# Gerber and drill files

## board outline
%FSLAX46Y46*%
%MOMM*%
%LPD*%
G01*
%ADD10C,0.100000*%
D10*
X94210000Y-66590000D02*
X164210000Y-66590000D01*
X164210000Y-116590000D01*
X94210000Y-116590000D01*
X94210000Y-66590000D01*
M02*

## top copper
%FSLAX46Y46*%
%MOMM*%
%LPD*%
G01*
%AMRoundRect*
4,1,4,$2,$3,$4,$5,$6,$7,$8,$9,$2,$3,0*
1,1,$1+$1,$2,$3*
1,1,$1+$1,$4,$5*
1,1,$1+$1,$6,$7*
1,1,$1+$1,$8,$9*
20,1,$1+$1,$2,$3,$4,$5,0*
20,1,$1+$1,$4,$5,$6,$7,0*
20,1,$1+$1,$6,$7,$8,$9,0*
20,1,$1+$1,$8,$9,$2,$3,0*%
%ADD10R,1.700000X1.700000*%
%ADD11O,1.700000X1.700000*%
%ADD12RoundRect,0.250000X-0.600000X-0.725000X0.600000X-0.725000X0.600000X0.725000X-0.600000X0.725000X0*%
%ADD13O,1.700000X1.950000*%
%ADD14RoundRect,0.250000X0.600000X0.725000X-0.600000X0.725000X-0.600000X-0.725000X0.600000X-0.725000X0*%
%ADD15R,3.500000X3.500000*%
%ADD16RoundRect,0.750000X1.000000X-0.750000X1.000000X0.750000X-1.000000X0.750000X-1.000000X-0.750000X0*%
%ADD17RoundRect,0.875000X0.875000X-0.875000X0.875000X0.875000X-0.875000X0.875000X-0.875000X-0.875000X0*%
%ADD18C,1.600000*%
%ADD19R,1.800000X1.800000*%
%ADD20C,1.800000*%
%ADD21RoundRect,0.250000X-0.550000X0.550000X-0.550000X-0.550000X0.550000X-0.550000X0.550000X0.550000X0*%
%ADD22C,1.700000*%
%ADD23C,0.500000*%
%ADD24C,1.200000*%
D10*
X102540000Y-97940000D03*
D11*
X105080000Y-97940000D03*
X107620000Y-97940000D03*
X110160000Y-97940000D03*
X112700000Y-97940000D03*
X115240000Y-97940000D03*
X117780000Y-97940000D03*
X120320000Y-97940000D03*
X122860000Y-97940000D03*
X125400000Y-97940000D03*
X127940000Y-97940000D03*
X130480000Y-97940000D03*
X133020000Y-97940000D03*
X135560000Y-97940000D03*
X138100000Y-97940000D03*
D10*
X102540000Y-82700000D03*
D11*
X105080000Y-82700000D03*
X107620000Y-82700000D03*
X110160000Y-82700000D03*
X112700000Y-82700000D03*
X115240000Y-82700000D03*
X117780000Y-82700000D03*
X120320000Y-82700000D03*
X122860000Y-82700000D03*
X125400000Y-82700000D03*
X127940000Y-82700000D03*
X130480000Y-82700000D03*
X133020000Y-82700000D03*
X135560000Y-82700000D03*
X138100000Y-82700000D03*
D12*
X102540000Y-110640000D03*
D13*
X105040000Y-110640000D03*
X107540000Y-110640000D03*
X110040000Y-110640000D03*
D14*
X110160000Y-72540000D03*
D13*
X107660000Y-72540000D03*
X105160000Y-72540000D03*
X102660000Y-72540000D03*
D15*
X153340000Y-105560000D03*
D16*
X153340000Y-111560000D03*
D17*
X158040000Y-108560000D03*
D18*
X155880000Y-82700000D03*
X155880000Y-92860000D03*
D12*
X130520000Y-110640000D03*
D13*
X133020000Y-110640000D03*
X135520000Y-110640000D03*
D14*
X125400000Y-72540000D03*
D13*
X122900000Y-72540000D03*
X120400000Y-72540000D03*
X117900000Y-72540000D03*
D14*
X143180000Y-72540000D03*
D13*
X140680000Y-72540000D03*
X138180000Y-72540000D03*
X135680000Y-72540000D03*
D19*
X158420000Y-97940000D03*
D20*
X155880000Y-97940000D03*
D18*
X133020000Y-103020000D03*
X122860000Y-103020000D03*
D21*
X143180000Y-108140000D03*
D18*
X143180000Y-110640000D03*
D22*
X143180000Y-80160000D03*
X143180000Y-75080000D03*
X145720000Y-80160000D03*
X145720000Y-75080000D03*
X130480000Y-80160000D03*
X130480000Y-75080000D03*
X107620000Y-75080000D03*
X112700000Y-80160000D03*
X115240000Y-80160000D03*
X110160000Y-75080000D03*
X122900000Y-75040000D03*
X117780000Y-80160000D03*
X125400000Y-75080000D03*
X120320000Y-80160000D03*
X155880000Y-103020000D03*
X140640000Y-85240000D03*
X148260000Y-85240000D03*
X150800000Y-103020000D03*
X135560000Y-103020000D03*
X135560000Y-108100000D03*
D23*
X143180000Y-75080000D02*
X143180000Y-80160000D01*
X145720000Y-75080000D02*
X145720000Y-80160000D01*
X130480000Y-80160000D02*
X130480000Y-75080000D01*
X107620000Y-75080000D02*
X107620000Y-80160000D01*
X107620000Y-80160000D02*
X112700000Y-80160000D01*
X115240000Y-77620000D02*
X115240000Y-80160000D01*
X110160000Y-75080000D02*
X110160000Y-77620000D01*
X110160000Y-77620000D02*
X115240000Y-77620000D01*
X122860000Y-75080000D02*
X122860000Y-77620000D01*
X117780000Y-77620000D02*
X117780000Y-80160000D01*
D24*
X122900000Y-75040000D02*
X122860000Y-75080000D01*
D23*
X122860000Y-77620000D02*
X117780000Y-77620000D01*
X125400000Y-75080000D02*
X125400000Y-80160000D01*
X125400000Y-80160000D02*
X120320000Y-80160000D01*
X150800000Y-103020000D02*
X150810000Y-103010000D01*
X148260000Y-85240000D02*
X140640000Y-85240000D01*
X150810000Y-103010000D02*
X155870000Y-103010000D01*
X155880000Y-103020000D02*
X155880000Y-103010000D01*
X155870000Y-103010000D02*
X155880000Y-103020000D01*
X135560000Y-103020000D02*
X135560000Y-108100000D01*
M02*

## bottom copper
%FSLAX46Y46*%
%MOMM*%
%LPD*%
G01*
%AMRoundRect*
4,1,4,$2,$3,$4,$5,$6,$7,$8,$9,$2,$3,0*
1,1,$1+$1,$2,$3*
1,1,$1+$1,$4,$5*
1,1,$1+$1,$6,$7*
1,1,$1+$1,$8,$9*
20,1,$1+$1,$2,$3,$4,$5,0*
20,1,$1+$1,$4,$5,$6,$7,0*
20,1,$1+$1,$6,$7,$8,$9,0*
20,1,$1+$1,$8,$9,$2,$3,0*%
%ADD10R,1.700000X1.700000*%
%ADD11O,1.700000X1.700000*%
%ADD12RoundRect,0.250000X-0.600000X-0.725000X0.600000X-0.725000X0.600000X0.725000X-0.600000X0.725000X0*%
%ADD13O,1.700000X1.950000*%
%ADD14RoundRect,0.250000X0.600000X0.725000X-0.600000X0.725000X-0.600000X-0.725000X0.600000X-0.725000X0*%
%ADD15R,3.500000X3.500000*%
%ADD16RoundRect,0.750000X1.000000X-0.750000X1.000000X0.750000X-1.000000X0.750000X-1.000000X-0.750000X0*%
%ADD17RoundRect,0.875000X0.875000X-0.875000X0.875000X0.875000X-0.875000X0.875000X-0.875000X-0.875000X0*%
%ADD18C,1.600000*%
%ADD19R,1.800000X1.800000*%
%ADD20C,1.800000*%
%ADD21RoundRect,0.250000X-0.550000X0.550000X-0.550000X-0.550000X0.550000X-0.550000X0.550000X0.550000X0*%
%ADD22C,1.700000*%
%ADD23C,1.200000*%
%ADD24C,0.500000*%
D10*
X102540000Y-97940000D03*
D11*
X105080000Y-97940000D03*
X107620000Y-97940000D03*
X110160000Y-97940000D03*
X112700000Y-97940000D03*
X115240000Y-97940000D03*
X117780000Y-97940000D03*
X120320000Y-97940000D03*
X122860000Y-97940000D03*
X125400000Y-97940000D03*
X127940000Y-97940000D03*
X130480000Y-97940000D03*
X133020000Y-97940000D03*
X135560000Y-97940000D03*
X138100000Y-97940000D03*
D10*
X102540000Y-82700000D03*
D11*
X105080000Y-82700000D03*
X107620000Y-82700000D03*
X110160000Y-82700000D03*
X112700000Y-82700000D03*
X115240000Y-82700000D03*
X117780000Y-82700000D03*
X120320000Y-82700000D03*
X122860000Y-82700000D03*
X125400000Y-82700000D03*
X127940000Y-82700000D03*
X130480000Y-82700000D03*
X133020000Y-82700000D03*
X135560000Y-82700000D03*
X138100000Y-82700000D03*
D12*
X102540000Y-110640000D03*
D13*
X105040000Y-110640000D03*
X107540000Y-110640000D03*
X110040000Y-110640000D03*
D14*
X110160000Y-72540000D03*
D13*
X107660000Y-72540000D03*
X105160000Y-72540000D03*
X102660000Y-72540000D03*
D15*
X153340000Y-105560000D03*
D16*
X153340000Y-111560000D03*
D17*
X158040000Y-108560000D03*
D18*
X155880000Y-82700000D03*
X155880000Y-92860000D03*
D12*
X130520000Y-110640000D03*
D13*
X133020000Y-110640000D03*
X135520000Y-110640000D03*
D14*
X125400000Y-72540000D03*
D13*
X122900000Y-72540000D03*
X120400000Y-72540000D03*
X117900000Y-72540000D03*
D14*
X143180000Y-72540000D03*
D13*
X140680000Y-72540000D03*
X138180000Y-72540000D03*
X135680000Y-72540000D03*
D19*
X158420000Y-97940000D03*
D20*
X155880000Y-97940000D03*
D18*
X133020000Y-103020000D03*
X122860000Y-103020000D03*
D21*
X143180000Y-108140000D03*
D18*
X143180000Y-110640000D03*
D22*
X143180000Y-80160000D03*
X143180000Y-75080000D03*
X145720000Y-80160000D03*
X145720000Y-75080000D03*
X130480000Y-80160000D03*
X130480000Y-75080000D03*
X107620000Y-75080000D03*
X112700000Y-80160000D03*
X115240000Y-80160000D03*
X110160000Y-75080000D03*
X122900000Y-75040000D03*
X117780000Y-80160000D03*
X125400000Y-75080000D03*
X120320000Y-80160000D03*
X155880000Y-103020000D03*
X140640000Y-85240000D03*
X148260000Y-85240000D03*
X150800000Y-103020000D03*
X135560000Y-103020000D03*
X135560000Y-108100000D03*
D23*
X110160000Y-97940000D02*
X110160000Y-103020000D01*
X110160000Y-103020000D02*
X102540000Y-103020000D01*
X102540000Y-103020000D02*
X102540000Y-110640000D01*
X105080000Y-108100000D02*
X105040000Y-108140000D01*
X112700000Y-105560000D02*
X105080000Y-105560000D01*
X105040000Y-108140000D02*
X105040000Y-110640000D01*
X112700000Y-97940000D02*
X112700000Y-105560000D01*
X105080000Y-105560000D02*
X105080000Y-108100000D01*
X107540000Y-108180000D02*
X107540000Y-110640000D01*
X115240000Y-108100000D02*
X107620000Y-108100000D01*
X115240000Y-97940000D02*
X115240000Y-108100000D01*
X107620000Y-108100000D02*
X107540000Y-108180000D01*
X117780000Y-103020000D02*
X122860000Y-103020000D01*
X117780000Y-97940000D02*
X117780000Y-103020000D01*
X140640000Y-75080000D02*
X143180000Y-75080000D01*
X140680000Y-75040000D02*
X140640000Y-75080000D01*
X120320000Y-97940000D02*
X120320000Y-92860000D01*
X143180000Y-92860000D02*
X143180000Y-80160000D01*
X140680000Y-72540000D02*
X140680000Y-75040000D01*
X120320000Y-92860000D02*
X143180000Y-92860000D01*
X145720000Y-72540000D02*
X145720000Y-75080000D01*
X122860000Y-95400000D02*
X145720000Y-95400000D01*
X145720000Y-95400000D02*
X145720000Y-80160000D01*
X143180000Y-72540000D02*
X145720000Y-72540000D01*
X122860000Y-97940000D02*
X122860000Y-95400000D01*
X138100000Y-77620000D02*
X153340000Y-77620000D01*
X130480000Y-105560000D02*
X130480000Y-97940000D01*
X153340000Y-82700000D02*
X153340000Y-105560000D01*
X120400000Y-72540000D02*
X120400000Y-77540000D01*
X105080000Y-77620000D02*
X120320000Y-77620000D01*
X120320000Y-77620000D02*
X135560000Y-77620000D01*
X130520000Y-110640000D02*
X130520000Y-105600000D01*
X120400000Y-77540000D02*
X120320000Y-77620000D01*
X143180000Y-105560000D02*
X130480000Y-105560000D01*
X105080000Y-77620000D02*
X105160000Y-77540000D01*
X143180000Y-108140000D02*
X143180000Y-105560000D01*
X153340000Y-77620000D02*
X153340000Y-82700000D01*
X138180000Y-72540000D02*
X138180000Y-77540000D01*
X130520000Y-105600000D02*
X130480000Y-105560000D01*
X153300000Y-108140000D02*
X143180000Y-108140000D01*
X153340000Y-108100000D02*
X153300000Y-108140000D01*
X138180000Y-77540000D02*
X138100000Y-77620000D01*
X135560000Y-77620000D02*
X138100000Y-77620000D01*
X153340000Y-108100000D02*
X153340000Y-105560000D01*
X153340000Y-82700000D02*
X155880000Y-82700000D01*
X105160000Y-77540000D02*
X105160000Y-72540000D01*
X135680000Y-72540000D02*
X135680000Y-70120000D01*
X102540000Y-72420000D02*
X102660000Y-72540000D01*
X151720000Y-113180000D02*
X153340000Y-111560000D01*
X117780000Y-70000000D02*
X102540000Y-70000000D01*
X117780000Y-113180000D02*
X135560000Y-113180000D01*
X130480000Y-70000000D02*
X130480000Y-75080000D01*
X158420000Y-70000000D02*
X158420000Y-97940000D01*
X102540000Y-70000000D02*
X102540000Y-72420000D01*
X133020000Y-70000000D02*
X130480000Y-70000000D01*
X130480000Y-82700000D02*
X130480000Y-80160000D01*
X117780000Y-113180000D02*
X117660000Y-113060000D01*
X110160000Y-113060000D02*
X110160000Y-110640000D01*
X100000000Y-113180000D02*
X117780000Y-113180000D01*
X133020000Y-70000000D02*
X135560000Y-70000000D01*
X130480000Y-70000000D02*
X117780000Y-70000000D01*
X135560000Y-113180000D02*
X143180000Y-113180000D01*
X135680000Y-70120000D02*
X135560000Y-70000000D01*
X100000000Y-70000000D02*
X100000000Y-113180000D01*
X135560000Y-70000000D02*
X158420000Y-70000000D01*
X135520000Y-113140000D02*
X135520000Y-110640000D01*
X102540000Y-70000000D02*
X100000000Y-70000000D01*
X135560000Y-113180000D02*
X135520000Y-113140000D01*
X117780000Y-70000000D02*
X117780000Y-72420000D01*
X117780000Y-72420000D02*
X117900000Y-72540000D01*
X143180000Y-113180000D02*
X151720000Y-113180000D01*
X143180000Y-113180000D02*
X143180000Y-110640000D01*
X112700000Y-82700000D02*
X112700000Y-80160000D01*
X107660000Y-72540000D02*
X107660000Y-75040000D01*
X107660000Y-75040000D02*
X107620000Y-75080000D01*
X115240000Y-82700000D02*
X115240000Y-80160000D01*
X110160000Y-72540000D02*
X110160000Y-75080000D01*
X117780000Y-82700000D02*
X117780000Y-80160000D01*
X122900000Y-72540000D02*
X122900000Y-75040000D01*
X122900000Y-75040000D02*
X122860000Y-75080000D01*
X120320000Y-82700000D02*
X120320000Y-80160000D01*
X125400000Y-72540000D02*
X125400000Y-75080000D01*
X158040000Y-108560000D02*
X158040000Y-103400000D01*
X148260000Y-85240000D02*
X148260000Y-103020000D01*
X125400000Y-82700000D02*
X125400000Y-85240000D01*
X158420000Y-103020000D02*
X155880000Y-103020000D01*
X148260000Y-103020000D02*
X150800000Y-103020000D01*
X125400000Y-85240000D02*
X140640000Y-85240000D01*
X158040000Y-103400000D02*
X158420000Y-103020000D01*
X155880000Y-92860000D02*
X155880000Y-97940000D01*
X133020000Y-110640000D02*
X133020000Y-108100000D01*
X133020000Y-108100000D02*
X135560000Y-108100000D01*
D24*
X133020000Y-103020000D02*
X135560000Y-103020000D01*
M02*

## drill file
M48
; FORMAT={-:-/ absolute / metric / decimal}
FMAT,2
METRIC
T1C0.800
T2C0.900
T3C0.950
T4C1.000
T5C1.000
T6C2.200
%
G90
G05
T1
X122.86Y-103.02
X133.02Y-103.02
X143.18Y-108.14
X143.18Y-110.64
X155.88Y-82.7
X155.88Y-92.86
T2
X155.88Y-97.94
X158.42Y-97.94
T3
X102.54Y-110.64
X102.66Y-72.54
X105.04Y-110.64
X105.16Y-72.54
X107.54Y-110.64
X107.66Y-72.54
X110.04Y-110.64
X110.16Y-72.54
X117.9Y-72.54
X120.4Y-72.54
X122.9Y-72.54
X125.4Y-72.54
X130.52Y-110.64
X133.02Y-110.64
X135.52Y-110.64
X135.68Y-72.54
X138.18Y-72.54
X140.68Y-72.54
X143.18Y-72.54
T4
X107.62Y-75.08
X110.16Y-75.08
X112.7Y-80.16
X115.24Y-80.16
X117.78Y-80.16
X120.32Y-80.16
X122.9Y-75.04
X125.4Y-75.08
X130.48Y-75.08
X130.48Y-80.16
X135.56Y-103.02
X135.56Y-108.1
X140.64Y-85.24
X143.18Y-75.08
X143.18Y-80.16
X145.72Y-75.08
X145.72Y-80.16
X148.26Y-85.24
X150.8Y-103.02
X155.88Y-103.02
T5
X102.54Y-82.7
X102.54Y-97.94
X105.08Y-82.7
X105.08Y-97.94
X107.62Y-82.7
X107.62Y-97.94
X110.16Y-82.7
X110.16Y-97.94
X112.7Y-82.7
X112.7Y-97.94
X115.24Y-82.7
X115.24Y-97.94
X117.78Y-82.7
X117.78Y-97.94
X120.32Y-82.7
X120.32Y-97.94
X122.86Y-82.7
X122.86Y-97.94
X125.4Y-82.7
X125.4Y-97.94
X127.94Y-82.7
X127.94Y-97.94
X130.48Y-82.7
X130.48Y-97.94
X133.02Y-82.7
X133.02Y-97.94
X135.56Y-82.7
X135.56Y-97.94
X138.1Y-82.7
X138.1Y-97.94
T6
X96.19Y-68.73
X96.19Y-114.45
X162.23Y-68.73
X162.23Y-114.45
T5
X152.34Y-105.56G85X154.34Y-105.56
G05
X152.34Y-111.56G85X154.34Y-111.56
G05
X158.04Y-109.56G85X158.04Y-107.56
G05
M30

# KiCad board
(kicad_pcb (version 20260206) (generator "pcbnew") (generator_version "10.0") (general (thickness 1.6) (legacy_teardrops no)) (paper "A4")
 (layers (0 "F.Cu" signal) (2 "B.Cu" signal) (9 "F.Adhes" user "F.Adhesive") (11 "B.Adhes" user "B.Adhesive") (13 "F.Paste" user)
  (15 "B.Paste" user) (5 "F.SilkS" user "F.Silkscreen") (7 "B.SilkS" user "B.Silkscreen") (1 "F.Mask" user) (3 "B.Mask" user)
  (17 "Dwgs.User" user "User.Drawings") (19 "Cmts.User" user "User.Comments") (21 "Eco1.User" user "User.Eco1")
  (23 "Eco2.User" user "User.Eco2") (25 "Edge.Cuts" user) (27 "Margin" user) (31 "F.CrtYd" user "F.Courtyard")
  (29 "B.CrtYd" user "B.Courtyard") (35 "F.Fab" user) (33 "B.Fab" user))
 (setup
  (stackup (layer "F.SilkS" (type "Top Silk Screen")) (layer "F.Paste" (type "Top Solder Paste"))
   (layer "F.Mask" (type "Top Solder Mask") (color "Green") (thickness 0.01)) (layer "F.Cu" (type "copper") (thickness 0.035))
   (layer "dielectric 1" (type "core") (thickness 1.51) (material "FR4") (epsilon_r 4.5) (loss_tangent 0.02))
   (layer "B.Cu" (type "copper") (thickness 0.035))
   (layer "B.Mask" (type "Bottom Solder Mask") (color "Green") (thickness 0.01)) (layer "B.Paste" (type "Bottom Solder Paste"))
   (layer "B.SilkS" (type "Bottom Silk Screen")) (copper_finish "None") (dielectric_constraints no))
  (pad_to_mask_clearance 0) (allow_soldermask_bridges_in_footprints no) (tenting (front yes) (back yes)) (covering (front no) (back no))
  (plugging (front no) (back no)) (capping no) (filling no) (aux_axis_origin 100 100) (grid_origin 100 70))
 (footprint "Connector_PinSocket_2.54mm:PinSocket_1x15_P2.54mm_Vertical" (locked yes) (layer "F.Cu") (at 102.54 97.94 90)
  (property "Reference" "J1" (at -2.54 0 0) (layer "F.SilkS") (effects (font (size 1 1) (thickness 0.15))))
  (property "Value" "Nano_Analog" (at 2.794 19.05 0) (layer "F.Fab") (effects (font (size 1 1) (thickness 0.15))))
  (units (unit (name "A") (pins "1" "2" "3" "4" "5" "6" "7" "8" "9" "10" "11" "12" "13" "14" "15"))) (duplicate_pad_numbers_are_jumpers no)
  (pad "1" thru_hole rect (at 0 0 90) (size 1.7 1.7) (drill 1) (layers "*.Cu" "*.Mask") (remove_unused_layers no) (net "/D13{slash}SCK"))
  (pad "2" thru_hole oval (at 0 2.54 90) (size 1.7 1.7) (drill 1) (layers "*.Cu" "*.Mask") (remove_unused_layers no) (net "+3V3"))
  (pad "3" thru_hole oval (at 0 5.08 90) (size 1.7 1.7) (drill 1) (layers "*.Cu" "*.Mask") (remove_unused_layers no) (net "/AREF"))
  (pad "4" thru_hole oval (at 0 7.62 90) (size 1.7 1.7) (drill 1) (layers "*.Cu" "*.Mask") (remove_unused_layers no) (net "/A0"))
  (pad "5" thru_hole oval (at 0 10.16 90) (size 1.7 1.7) (drill 1) (layers "*.Cu" "*.Mask") (remove_unused_layers no) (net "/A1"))
  (pad "6" thru_hole oval (at 0 12.7 90) (size 1.7 1.7) (drill 1) (layers "*.Cu" "*.Mask") (remove_unused_layers no) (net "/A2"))
  (pad "7" thru_hole oval (at 0 15.24 90) (size 1.7 1.7) (drill 1) (layers "*.Cu" "*.Mask") (remove_unused_layers no) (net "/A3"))
  (pad "8" thru_hole oval (at 0 17.78 90) (size 1.7 1.7) (drill 1) (layers "*.Cu" "*.Mask") (remove_unused_layers no) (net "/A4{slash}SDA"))
  (pad "9" thru_hole oval (at 0 20.32 90) (size 1.7 1.7) (drill 1) (layers "*.Cu" "*.Mask") (remove_unused_layers no) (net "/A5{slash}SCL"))
  (pad "10" thru_hole oval (at 0 22.86 90) (size 1.7 1.7) (drill 1) (layers "*.Cu" "*.Mask") (remove_unused_layers no) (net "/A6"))
  (pad "11" thru_hole oval (at 0 25.4 90) (size 1.7 1.7) (drill 1) (layers "*.Cu" "*.Mask") (remove_unused_layers no) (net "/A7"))
  (pad "12" thru_hole oval (at 0 27.94 90) (size 1.7 1.7) (drill 1) (layers "*.Cu" "*.Mask") (remove_unused_layers no) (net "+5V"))
  (pad "13" thru_hole oval (at 0 30.48 90) (size 1.7 1.7) (drill 1) (layers "*.Cu" "*.Mask") (remove_unused_layers no)
   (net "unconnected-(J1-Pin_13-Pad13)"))
  (pad "14" thru_hole oval (at 0 33.02 90) (size 1.7 1.7) (drill 1) (layers "*.Cu" "*.Mask") (remove_unused_layers no)
   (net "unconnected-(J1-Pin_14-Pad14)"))
  (pad "15" thru_hole oval (at 0 35.56 90) (size 1.7 1.7) (drill 1) (layers "*.Cu" "*.Mask") (remove_unused_layers no) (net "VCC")))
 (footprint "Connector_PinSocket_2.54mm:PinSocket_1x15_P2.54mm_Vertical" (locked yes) (layer "F.Cu") (at 102.54 82.7 90)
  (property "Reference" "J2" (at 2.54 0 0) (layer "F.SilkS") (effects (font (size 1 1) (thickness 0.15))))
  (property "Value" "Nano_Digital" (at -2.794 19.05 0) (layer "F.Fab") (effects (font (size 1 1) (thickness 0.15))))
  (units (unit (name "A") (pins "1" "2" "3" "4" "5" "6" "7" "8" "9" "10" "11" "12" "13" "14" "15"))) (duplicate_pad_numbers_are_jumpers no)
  (pad "1" thru_hole rect (at 0 0 90) (size 1.7 1.7) (drill 1) (layers "*.Cu" "*.Mask") (remove_unused_layers no) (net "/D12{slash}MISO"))
  (pad "2" thru_hole oval (at 0 2.54 90) (size 1.7 1.7) (drill 1) (layers "*.Cu" "*.Mask") (remove_unused_layers no)
   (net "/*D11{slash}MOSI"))
  (pad "3" thru_hole oval (at 0 5.08 90) (size 1.7 1.7) (drill 1) (layers "*.Cu" "*.Mask") (remove_unused_layers no) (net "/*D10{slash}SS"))
  (pad "4" thru_hole oval (at 0 7.62 90) (size 1.7 1.7) (drill 1) (layers "*.Cu" "*.Mask") (remove_unused_layers no) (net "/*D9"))
  (pad "5" thru_hole oval (at 0 10.16 90) (size 1.7 1.7) (drill 1) (layers "*.Cu" "*.Mask") (remove_unused_layers no) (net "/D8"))
  (pad "6" thru_hole oval (at 0 12.7 90) (size 1.7 1.7) (drill 1) (layers "*.Cu" "*.Mask") (remove_unused_layers no) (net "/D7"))
  (pad "7" thru_hole oval (at 0 15.24 90) (size 1.7 1.7) (drill 1) (layers "*.Cu" "*.Mask") (remove_unused_layers no) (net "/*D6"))
  (pad "8" thru_hole oval (at 0 17.78 90) (size 1.7 1.7) (drill 1) (layers "*.Cu" "*.Mask") (remove_unused_layers no) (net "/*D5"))
  (pad "9" thru_hole oval (at 0 20.32 90) (size 1.7 1.7) (drill 1) (layers "*.Cu" "*.Mask") (remove_unused_layers no) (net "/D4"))
  (pad "10" thru_hole oval (at 0 22.86 90) (size 1.7 1.7) (drill 1) (layers "*.Cu" "*.Mask") (remove_unused_layers no) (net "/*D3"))
  (pad "11" thru_hole oval (at 0 25.4 90) (size 1.7 1.7) (drill 1) (layers "*.Cu" "*.Mask") (remove_unused_layers no) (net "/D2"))
  (pad "12" thru_hole oval (at 0 27.94 90) (size 1.7 1.7) (drill 1) (layers "*.Cu" "*.Mask") (remove_unused_layers no) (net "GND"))
  (pad "13" thru_hole oval (at 0 30.48 90) (size 1.7 1.7) (drill 1) (layers "*.Cu" "*.Mask") (remove_unused_layers no)
   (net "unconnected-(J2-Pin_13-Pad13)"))
  (pad "14" thru_hole oval (at 0 33.02 90) (size 1.7 1.7) (drill 1) (layers "*.Cu" "*.Mask") (remove_unused_layers no) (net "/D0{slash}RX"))
  (pad "15" thru_hole oval (at 0 35.56 90) (size 1.7 1.7) (drill 1) (layers "*.Cu" "*.Mask") (remove_unused_layers no) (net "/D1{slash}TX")))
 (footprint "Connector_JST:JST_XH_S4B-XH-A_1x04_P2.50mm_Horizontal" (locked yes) (layer "F.Cu") (at 102.54 110.64)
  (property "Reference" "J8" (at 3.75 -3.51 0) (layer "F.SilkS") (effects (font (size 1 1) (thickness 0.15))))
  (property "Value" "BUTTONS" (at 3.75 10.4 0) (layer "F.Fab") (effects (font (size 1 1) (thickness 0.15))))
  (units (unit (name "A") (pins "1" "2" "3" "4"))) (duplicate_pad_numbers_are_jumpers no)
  (pad "1" thru_hole roundrect (at 0 0) (size 1.7 1.95) (drill 0.95) (layers "*.Cu" "*.Mask") (remove_unused_layers no)
   (roundrect_rratio 0.147059) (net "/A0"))
  (pad "2" thru_hole oval (at 2.5 0) (size 1.7 1.95) (drill 0.95) (layers "*.Cu" "*.Mask") (remove_unused_layers no) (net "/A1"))
  (pad "3" thru_hole oval (at 5 0) (size 1.7 1.95) (drill 0.95) (layers "*.Cu" "*.Mask") (remove_unused_layers no) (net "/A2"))
  (pad "4" thru_hole oval (at 7.5 0) (size 1.7 1.95) (drill 0.95) (layers "*.Cu" "*.Mask") (remove_unused_layers no) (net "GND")))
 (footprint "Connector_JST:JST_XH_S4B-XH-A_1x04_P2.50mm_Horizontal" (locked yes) (layer "F.Cu") (at 110.16 72.54 180)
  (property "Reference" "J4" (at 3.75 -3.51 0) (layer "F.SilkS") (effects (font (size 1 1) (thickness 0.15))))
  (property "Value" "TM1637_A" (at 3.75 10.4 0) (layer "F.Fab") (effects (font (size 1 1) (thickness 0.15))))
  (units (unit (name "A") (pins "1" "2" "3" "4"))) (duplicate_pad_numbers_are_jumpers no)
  (pad "1" thru_hole roundrect (at 0 0 180) (size 1.7 1.95) (drill 0.95) (layers "*.Cu" "*.Mask") (remove_unused_layers no)
   (roundrect_rratio 0.147059) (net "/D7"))
  (pad "2" thru_hole oval (at 2.5 0 180) (size 1.7 1.95) (drill 0.95) (layers "*.Cu" "*.Mask") (remove_unused_layers no) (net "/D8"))
  (pad "3" thru_hole oval (at 5 0 180) (size 1.7 1.95) (drill 0.95) (layers "*.Cu" "*.Mask") (remove_unused_layers no) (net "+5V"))
  (pad "4" thru_hole oval (at 7.5 0 180) (size 1.7 1.95) (drill 0.95) (layers "*.Cu" "*.Mask") (remove_unused_layers no) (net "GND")))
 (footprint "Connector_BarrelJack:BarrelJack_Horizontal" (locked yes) (layer "F.Cu") (at 153.34 105.56 90)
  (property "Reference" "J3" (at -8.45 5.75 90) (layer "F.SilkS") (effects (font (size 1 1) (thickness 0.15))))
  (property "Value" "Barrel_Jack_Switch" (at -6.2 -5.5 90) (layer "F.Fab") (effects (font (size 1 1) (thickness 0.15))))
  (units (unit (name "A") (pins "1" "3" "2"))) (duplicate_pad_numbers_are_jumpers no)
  (pad "1" thru_hole rect (at 0 0 90) (size 3.5 3.5) (drill oval 1 3) (layers "*.Cu" "*.Mask") (remove_unused_layers no) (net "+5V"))
  (pad "2" thru_hole roundrect (at -6 0 90) (size 3 3.5) (drill oval 1 3) (layers "*.Cu" "*.Mask") (remove_unused_layers no)
   (roundrect_rratio 0.25) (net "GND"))
  (pad "3" thru_hole roundrect (at -3 4.7 90) (size 3.5 3.5) (drill oval 3 1) (layers "*.Cu" "*.Mask") (remove_unused_layers no)
   (roundrect_rratio 0.25) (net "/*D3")))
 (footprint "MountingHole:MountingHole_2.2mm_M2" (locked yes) (layer "F.Cu") (at 162.23 68.73)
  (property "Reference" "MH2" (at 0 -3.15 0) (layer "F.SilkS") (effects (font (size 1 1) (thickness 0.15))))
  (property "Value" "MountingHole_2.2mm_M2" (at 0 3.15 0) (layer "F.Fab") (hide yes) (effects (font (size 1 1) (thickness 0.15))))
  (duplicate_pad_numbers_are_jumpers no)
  (pad "" np_thru_hole circle (at 0 0) (size 2.2 2.2) (drill 2.2) (layers "*.Cu" "*.Mask")))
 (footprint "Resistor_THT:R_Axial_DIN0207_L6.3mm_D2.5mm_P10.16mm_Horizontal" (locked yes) (layer "F.Cu") (at 155.88 82.7 -90)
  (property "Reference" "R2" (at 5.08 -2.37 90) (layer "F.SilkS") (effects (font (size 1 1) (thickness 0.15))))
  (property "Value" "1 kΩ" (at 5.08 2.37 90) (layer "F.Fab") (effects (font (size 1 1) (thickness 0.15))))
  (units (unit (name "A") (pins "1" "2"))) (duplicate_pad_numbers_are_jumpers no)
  (pad "1" thru_hole circle (at 0 0 270) (size 1.6 1.6) (drill 0.8) (layers "*.Cu" "*.Mask") (remove_unused_layers no) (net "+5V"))
  (pad "2" thru_hole circle (at 10.16 0 270) (size 1.6 1.6) (drill 0.8) (layers "*.Cu" "*.Mask") (remove_unused_layers no)
   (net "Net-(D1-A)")))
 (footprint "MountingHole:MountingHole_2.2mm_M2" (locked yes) (layer "F.Cu") (at 162.23 114.45)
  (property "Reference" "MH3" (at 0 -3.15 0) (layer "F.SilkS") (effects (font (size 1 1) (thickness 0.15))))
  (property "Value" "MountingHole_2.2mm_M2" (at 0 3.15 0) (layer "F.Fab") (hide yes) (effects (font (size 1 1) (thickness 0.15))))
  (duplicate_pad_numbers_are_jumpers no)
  (pad "" np_thru_hole circle (at 0 0) (size 2.2 2.2) (drill 2.2) (layers "*.Cu" "*.Mask")))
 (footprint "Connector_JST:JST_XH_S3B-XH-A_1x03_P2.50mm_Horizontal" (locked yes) (layer "F.Cu") (at 130.52 110.64)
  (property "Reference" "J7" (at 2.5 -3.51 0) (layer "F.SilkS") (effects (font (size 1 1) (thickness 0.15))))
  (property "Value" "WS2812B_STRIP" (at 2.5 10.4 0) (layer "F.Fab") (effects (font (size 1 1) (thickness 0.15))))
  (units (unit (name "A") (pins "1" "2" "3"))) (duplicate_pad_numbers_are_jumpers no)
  (pad "1" thru_hole roundrect (at 0 0) (size 1.7 1.95) (drill 0.95) (layers "*.Cu" "*.Mask") (remove_unused_layers no)
   (roundrect_rratio 0.147059) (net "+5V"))
  (pad "2" thru_hole oval (at 2.5 0) (size 1.7 1.95) (drill 0.95) (layers "*.Cu" "*.Mask") (remove_unused_layers no) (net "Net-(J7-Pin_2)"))
  (pad "3" thru_hole oval (at 5 0) (size 1.7 1.95) (drill 0.95) (layers "*.Cu" "*.Mask") (remove_unused_layers no) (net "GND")))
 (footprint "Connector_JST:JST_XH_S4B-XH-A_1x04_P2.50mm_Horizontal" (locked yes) (layer "F.Cu") (at 125.4 72.54 180)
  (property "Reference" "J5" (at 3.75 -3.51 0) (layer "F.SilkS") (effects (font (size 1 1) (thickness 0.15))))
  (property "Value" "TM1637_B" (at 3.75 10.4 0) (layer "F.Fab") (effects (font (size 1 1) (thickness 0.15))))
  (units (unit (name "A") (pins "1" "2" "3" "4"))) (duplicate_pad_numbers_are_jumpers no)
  (pad "1" thru_hole roundrect (at 0 0 180) (size 1.7 1.95) (drill 0.95) (layers "*.Cu" "*.Mask") (remove_unused_layers no)
   (roundrect_rratio 0.147059) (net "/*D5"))
  (pad "2" thru_hole oval (at 2.5 0 180) (size 1.7 1.95) (drill 0.95) (layers "*.Cu" "*.Mask") (remove_unused_layers no) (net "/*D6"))
  (pad "3" thru_hole oval (at 5 0 180) (size 1.7 1.95) (drill 0.95) (layers "*.Cu" "*.Mask") (remove_unused_layers no) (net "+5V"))
  (pad "4" thru_hole oval (at 7.5 0 180) (size 1.7 1.95) (drill 0.95) (layers "*.Cu" "*.Mask") (remove_unused_layers no) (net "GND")))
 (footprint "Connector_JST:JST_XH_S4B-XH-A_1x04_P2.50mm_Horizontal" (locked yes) (layer "F.Cu") (at 143.18 72.54 180)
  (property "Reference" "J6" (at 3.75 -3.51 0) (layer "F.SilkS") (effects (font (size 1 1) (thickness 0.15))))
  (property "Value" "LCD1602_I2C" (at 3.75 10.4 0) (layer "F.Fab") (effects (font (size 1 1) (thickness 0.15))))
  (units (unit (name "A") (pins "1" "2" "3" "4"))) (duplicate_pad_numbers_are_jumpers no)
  (pad "1" thru_hole roundrect (at 0 0 180) (size 1.7 1.95) (drill 0.95) (layers "*.Cu" "*.Mask") (remove_unused_layers no)
   (roundrect_rratio 0.147059) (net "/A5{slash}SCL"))
  (pad "2" thru_hole oval (at 2.5 0 180) (size 1.7 1.95) (drill 0.95) (layers "*.Cu" "*.Mask") (remove_unused_layers no)
   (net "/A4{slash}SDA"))
  (pad "3" thru_hole oval (at 5 0 180) (size 1.7 1.95) (drill 0.95) (layers "*.Cu" "*.Mask") (remove_unused_layers no) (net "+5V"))
  (pad "4" thru_hole oval (at 7.5 0 180) (size 1.7 1.95) (drill 0.95) (layers "*.Cu" "*.Mask") (remove_unused_layers no) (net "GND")))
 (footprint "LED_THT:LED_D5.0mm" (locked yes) (layer "F.Cu") (at 158.42 97.94 180)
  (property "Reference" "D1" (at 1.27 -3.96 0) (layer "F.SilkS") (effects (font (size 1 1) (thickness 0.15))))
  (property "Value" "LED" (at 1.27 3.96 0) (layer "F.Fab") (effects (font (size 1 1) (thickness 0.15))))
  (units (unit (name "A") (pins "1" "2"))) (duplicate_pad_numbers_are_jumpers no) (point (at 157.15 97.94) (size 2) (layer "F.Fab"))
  (pad "1" thru_hole rect (at 0 0 180) (size 1.8 1.8) (drill 0.9) (layers "*.Cu" "*.Mask") (remove_unused_layers no) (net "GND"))
  (pad "2" thru_hole circle (at 2.54 0 180) (size 1.8 1.8) (drill 0.9) (layers "*.Cu" "*.Mask") (remove_unused_layers no) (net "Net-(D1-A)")))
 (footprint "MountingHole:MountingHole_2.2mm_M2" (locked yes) (layer "F.Cu") (at 96.19 114.45)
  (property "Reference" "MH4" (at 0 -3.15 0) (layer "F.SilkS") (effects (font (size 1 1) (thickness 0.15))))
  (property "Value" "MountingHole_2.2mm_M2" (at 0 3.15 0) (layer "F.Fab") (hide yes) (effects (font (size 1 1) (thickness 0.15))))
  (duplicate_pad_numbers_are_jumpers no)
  (pad "" np_thru_hole circle (at 0 0) (size 2.2 2.2) (drill 2.2) (layers "*.Cu" "*.Mask")))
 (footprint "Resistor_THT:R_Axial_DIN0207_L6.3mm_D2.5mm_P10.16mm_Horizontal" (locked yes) (layer "F.Cu") (at 133.02 103.02 180)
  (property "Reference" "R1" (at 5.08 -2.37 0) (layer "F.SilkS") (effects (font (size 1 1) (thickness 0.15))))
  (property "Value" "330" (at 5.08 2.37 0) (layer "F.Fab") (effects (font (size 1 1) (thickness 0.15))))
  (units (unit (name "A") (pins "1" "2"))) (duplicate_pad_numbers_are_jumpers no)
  (pad "1" thru_hole circle (at 0 0 180) (size 1.6 1.6) (drill 0.8) (layers "*.Cu" "*.Mask") (remove_unused_layers no)
   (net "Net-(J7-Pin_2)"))
  (pad "2" thru_hole circle (at 10.16 0 180) (size 1.6 1.6) (drill 0.8) (layers "*.Cu" "*.Mask") (remove_unused_layers no) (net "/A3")))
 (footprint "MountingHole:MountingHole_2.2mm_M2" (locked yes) (layer "F.Cu") (at 96.19 68.73)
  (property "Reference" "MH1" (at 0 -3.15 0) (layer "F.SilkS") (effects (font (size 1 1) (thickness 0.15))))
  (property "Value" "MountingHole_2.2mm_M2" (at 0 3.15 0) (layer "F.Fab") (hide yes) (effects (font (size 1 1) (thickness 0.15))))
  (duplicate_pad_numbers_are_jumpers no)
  (pad "" np_thru_hole circle (at 0 0) (size 2.2 2.2) (drill 2.2) (layers "*.Cu" "*.Mask")))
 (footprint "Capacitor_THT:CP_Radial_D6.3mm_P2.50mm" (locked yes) (layer "F.Cu") (at 143.18 108.14 -90)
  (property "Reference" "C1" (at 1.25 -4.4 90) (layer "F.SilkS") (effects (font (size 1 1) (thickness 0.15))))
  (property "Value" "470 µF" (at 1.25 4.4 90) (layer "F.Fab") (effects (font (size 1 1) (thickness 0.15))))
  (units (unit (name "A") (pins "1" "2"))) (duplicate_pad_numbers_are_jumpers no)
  (pad "1" thru_hole roundrect (at 0 0 270) (size 1.6 1.6) (drill 0.8) (layers "*.Cu" "*.Mask") (remove_unused_layers no)
   (roundrect_rratio 0.15625) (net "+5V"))
  (pad "2" thru_hole circle (at 2.5 0 270) (size 1.6 1.6) (drill 0.8) (layers "*.Cu" "*.Mask") (remove_unused_layers no) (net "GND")))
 (gr_rect (start 94.21 66.59) (end 164.21 116.59) (stroke (width 0.1) (type solid)) (fill no) (locked yes) (layer "Edge.Cuts"))
 (segment (start 110.16 97.94) (end 110.16 103.02) (width 1.2) (layer "B.Cu") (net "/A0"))
 (segment (start 110.16 103.02) (end 102.54 103.02) (width 1.2) (layer "B.Cu") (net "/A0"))
 (segment (start 102.54 103.02) (end 102.54 110.64) (width 1.2) (layer "B.Cu") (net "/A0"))
 (segment (start 105.08 108.1) (end 105.04 108.14) (width 1.2) (layer "B.Cu") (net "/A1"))
 (segment (start 112.7 105.56) (end 105.08 105.56) (width 1.2) (layer "B.Cu") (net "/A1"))
 (segment (start 105.04 108.14) (end 105.04 110.64) (width 1.2) (layer "B.Cu") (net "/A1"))
 (segment (start 112.7 97.94) (end 112.7 105.56) (width 1.2) (layer "B.Cu") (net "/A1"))
 (segment (start 105.08 105.56) (end 105.08 108.1) (width 1.2) (layer "B.Cu") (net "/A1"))
 (segment (start 107.54 108.18) (end 107.54 110.64) (width 1.2) (layer "B.Cu") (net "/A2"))
 (segment (start 115.24 108.1) (end 107.62 108.1) (width 1.2) (layer "B.Cu") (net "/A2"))
 (segment (start 115.24 97.94) (end 115.24 108.1) (width 1.2) (layer "B.Cu") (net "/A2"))
 (segment (start 107.62 108.1) (end 107.54 108.18) (width 1.2) (layer "B.Cu") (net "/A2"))
 (segment (start 117.78 103.02) (end 122.86 103.02) (width 1.2) (layer "B.Cu") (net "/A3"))
 (segment (start 117.78 97.94) (end 117.78 103.02) (width 1.2) (layer "B.Cu") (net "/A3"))
 (segment (start 143.18 75.08) (end 143.18 80.16) (width 0.5) (layer "F.Cu") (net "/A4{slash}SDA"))
 (via (at 143.18 80.16) (size 1.7) (drill 1) (layers "F.Cu" "B.Cu") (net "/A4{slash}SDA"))
 (via (at 143.18 75.08) (size 1.7) (drill 1) (layers "F.Cu" "B.Cu") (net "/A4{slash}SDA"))
 (segment (start 140.64 75.08) (end 143.18 75.08) (width 1.2) (layer "B.Cu") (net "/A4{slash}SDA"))
 (segment (start 140.68 75.04) (end 140.64 75.08) (width 1.2) (layer "B.Cu") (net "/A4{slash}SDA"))
 (segment (start 120.32 97.94) (end 120.32 92.86) (width 1.2) (layer "B.Cu") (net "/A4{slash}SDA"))
 (segment (start 143.18 92.86) (end 143.18 80.16) (width 1.2) (layer "B.Cu") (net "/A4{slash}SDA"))
 (segment (start 140.68 72.54) (end 140.68 75.04) (width 1.2) (layer "B.Cu") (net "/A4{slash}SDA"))
 (segment (start 120.32 92.86) (end 143.18 92.86) (width 1.2) (layer "B.Cu") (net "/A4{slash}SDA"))
 (segment (start 145.72 75.08) (end 145.72 80.16) (width 0.5) (layer "F.Cu") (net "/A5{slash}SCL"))
 (via (at 145.72 80.16) (size 1.7) (drill 1) (layers "F.Cu" "B.Cu") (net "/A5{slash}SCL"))
 (via (at 145.72 75.08) (size 1.7) (drill 1) (layers "F.Cu" "B.Cu") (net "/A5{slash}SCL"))
 (segment (start 145.72 72.54) (end 145.72 75.08) (width 1.2) (layer "B.Cu") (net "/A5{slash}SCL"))
 (segment (start 122.86 95.4) (end 145.72 95.4) (width 1.2) (layer "B.Cu") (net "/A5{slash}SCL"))
 (segment (start 145.72 95.4) (end 145.72 80.16) (width 1.2) (layer "B.Cu") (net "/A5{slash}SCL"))
 (segment (start 143.18 72.54) (end 145.72 72.54) (width 1.2) (layer "B.Cu") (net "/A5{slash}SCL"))
 (segment (start 122.86 97.94) (end 122.86 95.4) (width 1.2) (layer "B.Cu") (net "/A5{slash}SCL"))
 (segment (start 138.1 77.62) (end 153.34 77.62) (width 1.2) (layer "B.Cu") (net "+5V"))
 (segment (start 130.48 105.56) (end 130.48 97.94) (width 1.2) (layer "B.Cu") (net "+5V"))
 (segment (start 153.34 82.7) (end 153.34 105.56) (width 1.2) (layer "B.Cu") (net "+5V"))
 (segment (start 120.4 72.54) (end 120.4 77.54) (width 1.2) (layer "B.Cu") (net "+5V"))
 (segment (start 105.08 77.62) (end 120.32 77.62) (width 1.2) (layer "B.Cu") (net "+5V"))
 (segment (start 120.32 77.62) (end 135.56 77.62) (width 1.2) (layer "B.Cu") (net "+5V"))
 (segment (start 130.52 110.64) (end 130.52 105.6) (width 1.2) (layer "B.Cu") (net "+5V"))
 (segment (start 120.4 77.54) (end 120.32 77.62) (width 1.2) (layer "B.Cu") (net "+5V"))
 (segment (start 143.18 105.56) (end 130.48 105.56) (width 1.2) (layer "B.Cu") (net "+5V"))
 (segment (start 105.08 77.62) (end 105.16 77.54) (width 1.2) (layer "B.Cu") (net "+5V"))
 (segment (start 143.18 108.14) (end 143.18 105.56) (width 1.2) (layer "B.Cu") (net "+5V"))
 (segment (start 153.34 77.62) (end 153.34 82.7) (width 1.2) (layer "B.Cu") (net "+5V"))
 (segment (start 138.18 72.54) (end 138.18 77.54) (width 1.2) (layer "B.Cu") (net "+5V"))
 (segment (start 130.52 105.6) (end 130.48 105.56) (width 1.2) (layer "B.Cu") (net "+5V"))
 (segment (start 153.3 108.14) (end 143.18 108.14) (width 1.2) (layer "B.Cu") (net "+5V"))
 (segment (start 153.34 108.1) (end 153.3 108.14) (width 1.2) (layer "B.Cu") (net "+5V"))
 (segment (start 138.18 77.54) (end 138.1 77.62) (width 1.2) (layer "B.Cu") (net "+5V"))
 (segment (start 135.56 77.62) (end 138.1 77.62) (width 1.2) (layer "B.Cu") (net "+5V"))
 (segment (start 153.34 108.1) (end 153.34 105.56) (width 1.2) (layer "B.Cu") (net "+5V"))
 (segment (start 153.34 82.7) (end 155.88 82.7) (width 1.2) (layer "B.Cu") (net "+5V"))
 (segment (start 105.16 77.54) (end 105.16 72.54) (width 1.2) (layer "B.Cu") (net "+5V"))
 (segment (start 130.48 80.16) (end 130.48 75.08) (width 0.5) (layer "F.Cu") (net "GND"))
 (via (at 130.48 80.16) (size 1.7) (drill 1) (layers "F.Cu" "B.Cu") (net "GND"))
 (via (at 130.48 75.08) (size 1.7) (drill 1) (layers "F.Cu" "B.Cu") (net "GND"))
 (segment (start 135.68 72.54) (end 135.68 70.12) (width 1.2) (layer "B.Cu") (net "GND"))
 (segment (start 102.54 72.42) (end 102.66 72.54) (width 1.2) (layer "B.Cu") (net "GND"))
 (segment (start 151.72 113.18) (end 153.34 111.56) (width 1.2) (layer "B.Cu") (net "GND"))
 (segment (start 117.78 70) (end 102.54 70) (width 1.2) (layer "B.Cu") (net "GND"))
 (segment (start 117.78 113.18) (end 135.56 113.18) (width 1.2) (layer "B.Cu") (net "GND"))
 (segment (start 130.48 70) (end 130.48 75.08) (width 1.2) (layer "B.Cu") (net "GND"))
 (segment (start 158.42 70) (end 158.42 97.94) (width 1.2) (layer "B.Cu") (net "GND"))
 (segment (start 102.54 70) (end 102.54 72.42) (width 1.2) (layer "B.Cu") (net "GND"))
 (segment (start 133.02 70) (end 130.48 70) (width 1.2) (layer "B.Cu") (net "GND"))
 (segment (start 130.48 82.7) (end 130.48 80.16) (width 1.2) (layer "B.Cu") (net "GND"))
 (segment (start 117.78 113.18) (end 117.66 113.06) (width 1.2) (layer "B.Cu") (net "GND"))
 (segment (start 110.16 113.06) (end 110.16 110.64) (width 1.2) (layer "B.Cu") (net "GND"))
 (segment (start 100 113.18) (end 117.78 113.18) (width 1.2) (layer "B.Cu") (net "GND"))
 (segment (start 133.02 70) (end 135.56 70) (width 1.2) (layer "B.Cu") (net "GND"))
 (segment (start 130.48 70) (end 117.78 70) (width 1.2) (layer "B.Cu") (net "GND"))
 (segment (start 135.56 113.18) (end 143.18 113.18) (width 1.2) (layer "B.Cu") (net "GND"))
 (segment (start 135.68 70.12) (end 135.56 70) (width 1.2) (layer "B.Cu") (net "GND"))
 (segment (start 100 70) (end 100 113.18) (width 1.2) (layer "B.Cu") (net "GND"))
 (segment (start 135.56 70) (end 158.42 70) (width 1.2) (layer "B.Cu") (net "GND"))
 (segment (start 135.52 113.14) (end 135.52 110.64) (width 1.2) (layer "B.Cu") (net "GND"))
 (segment (start 102.54 70) (end 100 70) (width 1.2) (layer "B.Cu") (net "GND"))
 (segment (start 135.56 113.18) (end 135.52 113.14) (width 1.2) (layer "B.Cu") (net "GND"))
 (segment (start 117.78 70) (end 117.78 72.42) (width 1.2) (layer "B.Cu") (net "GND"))
 (segment (start 117.78 72.42) (end 117.9 72.54) (width 1.2) (layer "B.Cu") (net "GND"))
 (segment (start 143.18 113.18) (end 151.72 113.18) (width 1.2) (layer "B.Cu") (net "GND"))
 (segment (start 143.18 113.18) (end 143.18 110.64) (width 1.2) (layer "B.Cu") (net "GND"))
 (segment (start 107.62 75.08) (end 107.62 80.16) (width 0.5) (layer "F.Cu") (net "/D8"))
 (segment (start 107.62 80.16) (end 112.7 80.16) (width 0.5) (layer "F.Cu") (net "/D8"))
 (via (at 107.62 75.08) (size 1.7) (drill 1) (layers "F.Cu" "B.Cu") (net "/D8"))
 (via (at 112.7 80.16) (size 1.7) (drill 1) (layers "F.Cu" "B.Cu") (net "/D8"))
 (segment (start 112.7 82.7) (end 112.7 80.16) (width 1.2) (layer "B.Cu") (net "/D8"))
 (segment (start 107.66 72.54) (end 107.66 75.04) (width 1.2) (layer "B.Cu") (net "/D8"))
 (segment (start 107.66 75.04) (end 107.62 75.08) (width 1.2) (layer "B.Cu") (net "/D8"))
 (segment (start 115.24 77.62) (end 115.24 80.16) (width 0.5) (layer "F.Cu") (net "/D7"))
 (segment (start 110.16 75.08) (end 110.16 77.62) (width 0.5) (layer "F.Cu") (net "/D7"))
 (segment (start 110.16 77.62) (end 115.24 77.62) (width 0.5) (layer "F.Cu") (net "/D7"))
 (via (at 115.24 80.16) (size 1.7) (drill 1) (layers "F.Cu" "B.Cu") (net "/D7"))
 (via (at 110.16 75.08) (size 1.7) (drill 1) (layers "F.Cu" "B.Cu") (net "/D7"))
 (segment (start 115.24 82.7) (end 115.24 80.16) (width 1.2) (layer "B.Cu") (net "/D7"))
 (segment (start 110.16 72.54) (end 110.16 75.08) (width 1.2) (layer "B.Cu") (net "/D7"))
 (segment (start 122.86 75.08) (end 122.86 77.62) (width 0.5) (layer "F.Cu") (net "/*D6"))
 (segment (start 117.78 77.62) (end 117.78 80.16) (width 0.5) (layer "F.Cu") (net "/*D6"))
 (segment (start 122.9 75.04) (end 122.86 75.08) (width 1.2) (layer "F.Cu") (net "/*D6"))
 (segment (start 122.86 77.62) (end 117.78 77.62) (width 0.5) (layer "F.Cu") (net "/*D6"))
 (via (at 122.9 75.04) (size 1.7) (drill 1) (layers "F.Cu" "B.Cu") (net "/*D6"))
 (via (at 117.78 80.16) (size 1.7) (drill 1) (layers "F.Cu" "B.Cu") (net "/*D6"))
 (segment (start 117.78 82.7) (end 117.78 80.16) (width 1.2) (layer "B.Cu") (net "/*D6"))
 (segment (start 122.9 72.54) (end 122.9 75.04) (width 1.2) (layer "B.Cu") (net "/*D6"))
 (segment (start 122.9 75.04) (end 122.86 75.08) (width 1.2) (layer "B.Cu") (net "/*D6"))
 (segment (start 125.4 75.08) (end 125.4 80.16) (width 0.5) (layer "F.Cu") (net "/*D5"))
 (segment (start 125.4 80.16) (end 120.32 80.16) (width 0.5) (layer "F.Cu") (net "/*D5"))
 (via (at 125.4 75.08) (size 1.7) (drill 1) (layers "F.Cu" "B.Cu") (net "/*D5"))
 (via (at 120.32 80.16) (size 1.7) (drill 1) (layers "F.Cu" "B.Cu") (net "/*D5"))
 (segment (start 120.32 82.7) (end 120.32 80.16) (width 1.2) (layer "B.Cu") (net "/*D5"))
 (segment (start 125.4 72.54) (end 125.4 75.08) (width 1.2) (layer "B.Cu") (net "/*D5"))
 (segment (start 150.8 103.02) (end 150.81 103.01) (width 0.5) (layer "F.Cu") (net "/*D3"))
 (segment (start 148.26 85.24) (end 140.64 85.24) (width 0.5) (layer "F.Cu") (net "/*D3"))
 (segment (start 150.81 103.01) (end 155.87 103.01) (width 0.5) (layer "F.Cu") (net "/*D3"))
 (segment (start 155.88 103.02) (end 155.88 103.01) (width 0.5) (layer "F.Cu") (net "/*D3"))
 (segment (start 155.87 103.01) (end 155.88 103.02) (width 0.5) (layer "F.Cu") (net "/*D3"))
 (via (at 155.88 103.02) (size 1.7) (drill 1) (layers "F.Cu" "B.Cu") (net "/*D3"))
 (via (at 140.64 85.24) (size 1.7) (drill 1) (layers "F.Cu" "B.Cu") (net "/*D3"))
 (via (at 148.26 85.24) (size 1.7) (drill 1) (layers "F.Cu" "B.Cu") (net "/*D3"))
 (via (at 150.8 103.02) (size 1.7) (drill 1) (layers "F.Cu" "B.Cu") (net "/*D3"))
 (segment (start 158.04 108.56) (end 158.04 103.4) (width 1.2) (layer "B.Cu") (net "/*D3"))
 (segment (start 148.26 85.24) (end 148.26 103.02) (width 1.2) (layer "B.Cu") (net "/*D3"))
 (segment (start 125.4 82.7) (end 125.4 85.24) (width 1.2) (layer "B.Cu") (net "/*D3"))
 (segment (start 158.42 103.02) (end 155.88 103.02) (width 1.2) (layer "B.Cu") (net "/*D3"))
 (segment (start 148.26 103.02) (end 150.8 103.02) (width 1.2) (layer "B.Cu") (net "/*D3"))
 (segment (start 125.4 85.24) (end 140.64 85.24) (width 1.2) (layer "B.Cu") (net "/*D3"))
 (segment (start 158.04 103.4) (end 158.42 103.02) (width 1.2) (layer "B.Cu") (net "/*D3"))
 (segment (start 155.88 92.86) (end 155.88 97.94) (width 1.2) (layer "B.Cu") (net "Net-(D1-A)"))
 (segment (start 135.56 103.02) (end 135.56 108.1) (width 0.5) (layer "F.Cu") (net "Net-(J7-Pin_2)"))
 (via (at 135.56 103.02) (size 1.7) (drill 1) (layers "F.Cu" "B.Cu") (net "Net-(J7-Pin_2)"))
 (via (at 135.56 108.1) (size 1.7) (drill 1) (layers "F.Cu" "B.Cu") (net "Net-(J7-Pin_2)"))
 (segment (start 133.02 110.64) (end 133.02 108.1) (width 1.2) (layer "B.Cu") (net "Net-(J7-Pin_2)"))
 (segment (start 133.02 108.1) (end 135.56 108.1) (width 1.2) (layer "B.Cu") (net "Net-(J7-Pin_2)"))
 (segment (start 133.02 103.02) (end 135.56 103.02) (width 0.5) (layer "B.Cu") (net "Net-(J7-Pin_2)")))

